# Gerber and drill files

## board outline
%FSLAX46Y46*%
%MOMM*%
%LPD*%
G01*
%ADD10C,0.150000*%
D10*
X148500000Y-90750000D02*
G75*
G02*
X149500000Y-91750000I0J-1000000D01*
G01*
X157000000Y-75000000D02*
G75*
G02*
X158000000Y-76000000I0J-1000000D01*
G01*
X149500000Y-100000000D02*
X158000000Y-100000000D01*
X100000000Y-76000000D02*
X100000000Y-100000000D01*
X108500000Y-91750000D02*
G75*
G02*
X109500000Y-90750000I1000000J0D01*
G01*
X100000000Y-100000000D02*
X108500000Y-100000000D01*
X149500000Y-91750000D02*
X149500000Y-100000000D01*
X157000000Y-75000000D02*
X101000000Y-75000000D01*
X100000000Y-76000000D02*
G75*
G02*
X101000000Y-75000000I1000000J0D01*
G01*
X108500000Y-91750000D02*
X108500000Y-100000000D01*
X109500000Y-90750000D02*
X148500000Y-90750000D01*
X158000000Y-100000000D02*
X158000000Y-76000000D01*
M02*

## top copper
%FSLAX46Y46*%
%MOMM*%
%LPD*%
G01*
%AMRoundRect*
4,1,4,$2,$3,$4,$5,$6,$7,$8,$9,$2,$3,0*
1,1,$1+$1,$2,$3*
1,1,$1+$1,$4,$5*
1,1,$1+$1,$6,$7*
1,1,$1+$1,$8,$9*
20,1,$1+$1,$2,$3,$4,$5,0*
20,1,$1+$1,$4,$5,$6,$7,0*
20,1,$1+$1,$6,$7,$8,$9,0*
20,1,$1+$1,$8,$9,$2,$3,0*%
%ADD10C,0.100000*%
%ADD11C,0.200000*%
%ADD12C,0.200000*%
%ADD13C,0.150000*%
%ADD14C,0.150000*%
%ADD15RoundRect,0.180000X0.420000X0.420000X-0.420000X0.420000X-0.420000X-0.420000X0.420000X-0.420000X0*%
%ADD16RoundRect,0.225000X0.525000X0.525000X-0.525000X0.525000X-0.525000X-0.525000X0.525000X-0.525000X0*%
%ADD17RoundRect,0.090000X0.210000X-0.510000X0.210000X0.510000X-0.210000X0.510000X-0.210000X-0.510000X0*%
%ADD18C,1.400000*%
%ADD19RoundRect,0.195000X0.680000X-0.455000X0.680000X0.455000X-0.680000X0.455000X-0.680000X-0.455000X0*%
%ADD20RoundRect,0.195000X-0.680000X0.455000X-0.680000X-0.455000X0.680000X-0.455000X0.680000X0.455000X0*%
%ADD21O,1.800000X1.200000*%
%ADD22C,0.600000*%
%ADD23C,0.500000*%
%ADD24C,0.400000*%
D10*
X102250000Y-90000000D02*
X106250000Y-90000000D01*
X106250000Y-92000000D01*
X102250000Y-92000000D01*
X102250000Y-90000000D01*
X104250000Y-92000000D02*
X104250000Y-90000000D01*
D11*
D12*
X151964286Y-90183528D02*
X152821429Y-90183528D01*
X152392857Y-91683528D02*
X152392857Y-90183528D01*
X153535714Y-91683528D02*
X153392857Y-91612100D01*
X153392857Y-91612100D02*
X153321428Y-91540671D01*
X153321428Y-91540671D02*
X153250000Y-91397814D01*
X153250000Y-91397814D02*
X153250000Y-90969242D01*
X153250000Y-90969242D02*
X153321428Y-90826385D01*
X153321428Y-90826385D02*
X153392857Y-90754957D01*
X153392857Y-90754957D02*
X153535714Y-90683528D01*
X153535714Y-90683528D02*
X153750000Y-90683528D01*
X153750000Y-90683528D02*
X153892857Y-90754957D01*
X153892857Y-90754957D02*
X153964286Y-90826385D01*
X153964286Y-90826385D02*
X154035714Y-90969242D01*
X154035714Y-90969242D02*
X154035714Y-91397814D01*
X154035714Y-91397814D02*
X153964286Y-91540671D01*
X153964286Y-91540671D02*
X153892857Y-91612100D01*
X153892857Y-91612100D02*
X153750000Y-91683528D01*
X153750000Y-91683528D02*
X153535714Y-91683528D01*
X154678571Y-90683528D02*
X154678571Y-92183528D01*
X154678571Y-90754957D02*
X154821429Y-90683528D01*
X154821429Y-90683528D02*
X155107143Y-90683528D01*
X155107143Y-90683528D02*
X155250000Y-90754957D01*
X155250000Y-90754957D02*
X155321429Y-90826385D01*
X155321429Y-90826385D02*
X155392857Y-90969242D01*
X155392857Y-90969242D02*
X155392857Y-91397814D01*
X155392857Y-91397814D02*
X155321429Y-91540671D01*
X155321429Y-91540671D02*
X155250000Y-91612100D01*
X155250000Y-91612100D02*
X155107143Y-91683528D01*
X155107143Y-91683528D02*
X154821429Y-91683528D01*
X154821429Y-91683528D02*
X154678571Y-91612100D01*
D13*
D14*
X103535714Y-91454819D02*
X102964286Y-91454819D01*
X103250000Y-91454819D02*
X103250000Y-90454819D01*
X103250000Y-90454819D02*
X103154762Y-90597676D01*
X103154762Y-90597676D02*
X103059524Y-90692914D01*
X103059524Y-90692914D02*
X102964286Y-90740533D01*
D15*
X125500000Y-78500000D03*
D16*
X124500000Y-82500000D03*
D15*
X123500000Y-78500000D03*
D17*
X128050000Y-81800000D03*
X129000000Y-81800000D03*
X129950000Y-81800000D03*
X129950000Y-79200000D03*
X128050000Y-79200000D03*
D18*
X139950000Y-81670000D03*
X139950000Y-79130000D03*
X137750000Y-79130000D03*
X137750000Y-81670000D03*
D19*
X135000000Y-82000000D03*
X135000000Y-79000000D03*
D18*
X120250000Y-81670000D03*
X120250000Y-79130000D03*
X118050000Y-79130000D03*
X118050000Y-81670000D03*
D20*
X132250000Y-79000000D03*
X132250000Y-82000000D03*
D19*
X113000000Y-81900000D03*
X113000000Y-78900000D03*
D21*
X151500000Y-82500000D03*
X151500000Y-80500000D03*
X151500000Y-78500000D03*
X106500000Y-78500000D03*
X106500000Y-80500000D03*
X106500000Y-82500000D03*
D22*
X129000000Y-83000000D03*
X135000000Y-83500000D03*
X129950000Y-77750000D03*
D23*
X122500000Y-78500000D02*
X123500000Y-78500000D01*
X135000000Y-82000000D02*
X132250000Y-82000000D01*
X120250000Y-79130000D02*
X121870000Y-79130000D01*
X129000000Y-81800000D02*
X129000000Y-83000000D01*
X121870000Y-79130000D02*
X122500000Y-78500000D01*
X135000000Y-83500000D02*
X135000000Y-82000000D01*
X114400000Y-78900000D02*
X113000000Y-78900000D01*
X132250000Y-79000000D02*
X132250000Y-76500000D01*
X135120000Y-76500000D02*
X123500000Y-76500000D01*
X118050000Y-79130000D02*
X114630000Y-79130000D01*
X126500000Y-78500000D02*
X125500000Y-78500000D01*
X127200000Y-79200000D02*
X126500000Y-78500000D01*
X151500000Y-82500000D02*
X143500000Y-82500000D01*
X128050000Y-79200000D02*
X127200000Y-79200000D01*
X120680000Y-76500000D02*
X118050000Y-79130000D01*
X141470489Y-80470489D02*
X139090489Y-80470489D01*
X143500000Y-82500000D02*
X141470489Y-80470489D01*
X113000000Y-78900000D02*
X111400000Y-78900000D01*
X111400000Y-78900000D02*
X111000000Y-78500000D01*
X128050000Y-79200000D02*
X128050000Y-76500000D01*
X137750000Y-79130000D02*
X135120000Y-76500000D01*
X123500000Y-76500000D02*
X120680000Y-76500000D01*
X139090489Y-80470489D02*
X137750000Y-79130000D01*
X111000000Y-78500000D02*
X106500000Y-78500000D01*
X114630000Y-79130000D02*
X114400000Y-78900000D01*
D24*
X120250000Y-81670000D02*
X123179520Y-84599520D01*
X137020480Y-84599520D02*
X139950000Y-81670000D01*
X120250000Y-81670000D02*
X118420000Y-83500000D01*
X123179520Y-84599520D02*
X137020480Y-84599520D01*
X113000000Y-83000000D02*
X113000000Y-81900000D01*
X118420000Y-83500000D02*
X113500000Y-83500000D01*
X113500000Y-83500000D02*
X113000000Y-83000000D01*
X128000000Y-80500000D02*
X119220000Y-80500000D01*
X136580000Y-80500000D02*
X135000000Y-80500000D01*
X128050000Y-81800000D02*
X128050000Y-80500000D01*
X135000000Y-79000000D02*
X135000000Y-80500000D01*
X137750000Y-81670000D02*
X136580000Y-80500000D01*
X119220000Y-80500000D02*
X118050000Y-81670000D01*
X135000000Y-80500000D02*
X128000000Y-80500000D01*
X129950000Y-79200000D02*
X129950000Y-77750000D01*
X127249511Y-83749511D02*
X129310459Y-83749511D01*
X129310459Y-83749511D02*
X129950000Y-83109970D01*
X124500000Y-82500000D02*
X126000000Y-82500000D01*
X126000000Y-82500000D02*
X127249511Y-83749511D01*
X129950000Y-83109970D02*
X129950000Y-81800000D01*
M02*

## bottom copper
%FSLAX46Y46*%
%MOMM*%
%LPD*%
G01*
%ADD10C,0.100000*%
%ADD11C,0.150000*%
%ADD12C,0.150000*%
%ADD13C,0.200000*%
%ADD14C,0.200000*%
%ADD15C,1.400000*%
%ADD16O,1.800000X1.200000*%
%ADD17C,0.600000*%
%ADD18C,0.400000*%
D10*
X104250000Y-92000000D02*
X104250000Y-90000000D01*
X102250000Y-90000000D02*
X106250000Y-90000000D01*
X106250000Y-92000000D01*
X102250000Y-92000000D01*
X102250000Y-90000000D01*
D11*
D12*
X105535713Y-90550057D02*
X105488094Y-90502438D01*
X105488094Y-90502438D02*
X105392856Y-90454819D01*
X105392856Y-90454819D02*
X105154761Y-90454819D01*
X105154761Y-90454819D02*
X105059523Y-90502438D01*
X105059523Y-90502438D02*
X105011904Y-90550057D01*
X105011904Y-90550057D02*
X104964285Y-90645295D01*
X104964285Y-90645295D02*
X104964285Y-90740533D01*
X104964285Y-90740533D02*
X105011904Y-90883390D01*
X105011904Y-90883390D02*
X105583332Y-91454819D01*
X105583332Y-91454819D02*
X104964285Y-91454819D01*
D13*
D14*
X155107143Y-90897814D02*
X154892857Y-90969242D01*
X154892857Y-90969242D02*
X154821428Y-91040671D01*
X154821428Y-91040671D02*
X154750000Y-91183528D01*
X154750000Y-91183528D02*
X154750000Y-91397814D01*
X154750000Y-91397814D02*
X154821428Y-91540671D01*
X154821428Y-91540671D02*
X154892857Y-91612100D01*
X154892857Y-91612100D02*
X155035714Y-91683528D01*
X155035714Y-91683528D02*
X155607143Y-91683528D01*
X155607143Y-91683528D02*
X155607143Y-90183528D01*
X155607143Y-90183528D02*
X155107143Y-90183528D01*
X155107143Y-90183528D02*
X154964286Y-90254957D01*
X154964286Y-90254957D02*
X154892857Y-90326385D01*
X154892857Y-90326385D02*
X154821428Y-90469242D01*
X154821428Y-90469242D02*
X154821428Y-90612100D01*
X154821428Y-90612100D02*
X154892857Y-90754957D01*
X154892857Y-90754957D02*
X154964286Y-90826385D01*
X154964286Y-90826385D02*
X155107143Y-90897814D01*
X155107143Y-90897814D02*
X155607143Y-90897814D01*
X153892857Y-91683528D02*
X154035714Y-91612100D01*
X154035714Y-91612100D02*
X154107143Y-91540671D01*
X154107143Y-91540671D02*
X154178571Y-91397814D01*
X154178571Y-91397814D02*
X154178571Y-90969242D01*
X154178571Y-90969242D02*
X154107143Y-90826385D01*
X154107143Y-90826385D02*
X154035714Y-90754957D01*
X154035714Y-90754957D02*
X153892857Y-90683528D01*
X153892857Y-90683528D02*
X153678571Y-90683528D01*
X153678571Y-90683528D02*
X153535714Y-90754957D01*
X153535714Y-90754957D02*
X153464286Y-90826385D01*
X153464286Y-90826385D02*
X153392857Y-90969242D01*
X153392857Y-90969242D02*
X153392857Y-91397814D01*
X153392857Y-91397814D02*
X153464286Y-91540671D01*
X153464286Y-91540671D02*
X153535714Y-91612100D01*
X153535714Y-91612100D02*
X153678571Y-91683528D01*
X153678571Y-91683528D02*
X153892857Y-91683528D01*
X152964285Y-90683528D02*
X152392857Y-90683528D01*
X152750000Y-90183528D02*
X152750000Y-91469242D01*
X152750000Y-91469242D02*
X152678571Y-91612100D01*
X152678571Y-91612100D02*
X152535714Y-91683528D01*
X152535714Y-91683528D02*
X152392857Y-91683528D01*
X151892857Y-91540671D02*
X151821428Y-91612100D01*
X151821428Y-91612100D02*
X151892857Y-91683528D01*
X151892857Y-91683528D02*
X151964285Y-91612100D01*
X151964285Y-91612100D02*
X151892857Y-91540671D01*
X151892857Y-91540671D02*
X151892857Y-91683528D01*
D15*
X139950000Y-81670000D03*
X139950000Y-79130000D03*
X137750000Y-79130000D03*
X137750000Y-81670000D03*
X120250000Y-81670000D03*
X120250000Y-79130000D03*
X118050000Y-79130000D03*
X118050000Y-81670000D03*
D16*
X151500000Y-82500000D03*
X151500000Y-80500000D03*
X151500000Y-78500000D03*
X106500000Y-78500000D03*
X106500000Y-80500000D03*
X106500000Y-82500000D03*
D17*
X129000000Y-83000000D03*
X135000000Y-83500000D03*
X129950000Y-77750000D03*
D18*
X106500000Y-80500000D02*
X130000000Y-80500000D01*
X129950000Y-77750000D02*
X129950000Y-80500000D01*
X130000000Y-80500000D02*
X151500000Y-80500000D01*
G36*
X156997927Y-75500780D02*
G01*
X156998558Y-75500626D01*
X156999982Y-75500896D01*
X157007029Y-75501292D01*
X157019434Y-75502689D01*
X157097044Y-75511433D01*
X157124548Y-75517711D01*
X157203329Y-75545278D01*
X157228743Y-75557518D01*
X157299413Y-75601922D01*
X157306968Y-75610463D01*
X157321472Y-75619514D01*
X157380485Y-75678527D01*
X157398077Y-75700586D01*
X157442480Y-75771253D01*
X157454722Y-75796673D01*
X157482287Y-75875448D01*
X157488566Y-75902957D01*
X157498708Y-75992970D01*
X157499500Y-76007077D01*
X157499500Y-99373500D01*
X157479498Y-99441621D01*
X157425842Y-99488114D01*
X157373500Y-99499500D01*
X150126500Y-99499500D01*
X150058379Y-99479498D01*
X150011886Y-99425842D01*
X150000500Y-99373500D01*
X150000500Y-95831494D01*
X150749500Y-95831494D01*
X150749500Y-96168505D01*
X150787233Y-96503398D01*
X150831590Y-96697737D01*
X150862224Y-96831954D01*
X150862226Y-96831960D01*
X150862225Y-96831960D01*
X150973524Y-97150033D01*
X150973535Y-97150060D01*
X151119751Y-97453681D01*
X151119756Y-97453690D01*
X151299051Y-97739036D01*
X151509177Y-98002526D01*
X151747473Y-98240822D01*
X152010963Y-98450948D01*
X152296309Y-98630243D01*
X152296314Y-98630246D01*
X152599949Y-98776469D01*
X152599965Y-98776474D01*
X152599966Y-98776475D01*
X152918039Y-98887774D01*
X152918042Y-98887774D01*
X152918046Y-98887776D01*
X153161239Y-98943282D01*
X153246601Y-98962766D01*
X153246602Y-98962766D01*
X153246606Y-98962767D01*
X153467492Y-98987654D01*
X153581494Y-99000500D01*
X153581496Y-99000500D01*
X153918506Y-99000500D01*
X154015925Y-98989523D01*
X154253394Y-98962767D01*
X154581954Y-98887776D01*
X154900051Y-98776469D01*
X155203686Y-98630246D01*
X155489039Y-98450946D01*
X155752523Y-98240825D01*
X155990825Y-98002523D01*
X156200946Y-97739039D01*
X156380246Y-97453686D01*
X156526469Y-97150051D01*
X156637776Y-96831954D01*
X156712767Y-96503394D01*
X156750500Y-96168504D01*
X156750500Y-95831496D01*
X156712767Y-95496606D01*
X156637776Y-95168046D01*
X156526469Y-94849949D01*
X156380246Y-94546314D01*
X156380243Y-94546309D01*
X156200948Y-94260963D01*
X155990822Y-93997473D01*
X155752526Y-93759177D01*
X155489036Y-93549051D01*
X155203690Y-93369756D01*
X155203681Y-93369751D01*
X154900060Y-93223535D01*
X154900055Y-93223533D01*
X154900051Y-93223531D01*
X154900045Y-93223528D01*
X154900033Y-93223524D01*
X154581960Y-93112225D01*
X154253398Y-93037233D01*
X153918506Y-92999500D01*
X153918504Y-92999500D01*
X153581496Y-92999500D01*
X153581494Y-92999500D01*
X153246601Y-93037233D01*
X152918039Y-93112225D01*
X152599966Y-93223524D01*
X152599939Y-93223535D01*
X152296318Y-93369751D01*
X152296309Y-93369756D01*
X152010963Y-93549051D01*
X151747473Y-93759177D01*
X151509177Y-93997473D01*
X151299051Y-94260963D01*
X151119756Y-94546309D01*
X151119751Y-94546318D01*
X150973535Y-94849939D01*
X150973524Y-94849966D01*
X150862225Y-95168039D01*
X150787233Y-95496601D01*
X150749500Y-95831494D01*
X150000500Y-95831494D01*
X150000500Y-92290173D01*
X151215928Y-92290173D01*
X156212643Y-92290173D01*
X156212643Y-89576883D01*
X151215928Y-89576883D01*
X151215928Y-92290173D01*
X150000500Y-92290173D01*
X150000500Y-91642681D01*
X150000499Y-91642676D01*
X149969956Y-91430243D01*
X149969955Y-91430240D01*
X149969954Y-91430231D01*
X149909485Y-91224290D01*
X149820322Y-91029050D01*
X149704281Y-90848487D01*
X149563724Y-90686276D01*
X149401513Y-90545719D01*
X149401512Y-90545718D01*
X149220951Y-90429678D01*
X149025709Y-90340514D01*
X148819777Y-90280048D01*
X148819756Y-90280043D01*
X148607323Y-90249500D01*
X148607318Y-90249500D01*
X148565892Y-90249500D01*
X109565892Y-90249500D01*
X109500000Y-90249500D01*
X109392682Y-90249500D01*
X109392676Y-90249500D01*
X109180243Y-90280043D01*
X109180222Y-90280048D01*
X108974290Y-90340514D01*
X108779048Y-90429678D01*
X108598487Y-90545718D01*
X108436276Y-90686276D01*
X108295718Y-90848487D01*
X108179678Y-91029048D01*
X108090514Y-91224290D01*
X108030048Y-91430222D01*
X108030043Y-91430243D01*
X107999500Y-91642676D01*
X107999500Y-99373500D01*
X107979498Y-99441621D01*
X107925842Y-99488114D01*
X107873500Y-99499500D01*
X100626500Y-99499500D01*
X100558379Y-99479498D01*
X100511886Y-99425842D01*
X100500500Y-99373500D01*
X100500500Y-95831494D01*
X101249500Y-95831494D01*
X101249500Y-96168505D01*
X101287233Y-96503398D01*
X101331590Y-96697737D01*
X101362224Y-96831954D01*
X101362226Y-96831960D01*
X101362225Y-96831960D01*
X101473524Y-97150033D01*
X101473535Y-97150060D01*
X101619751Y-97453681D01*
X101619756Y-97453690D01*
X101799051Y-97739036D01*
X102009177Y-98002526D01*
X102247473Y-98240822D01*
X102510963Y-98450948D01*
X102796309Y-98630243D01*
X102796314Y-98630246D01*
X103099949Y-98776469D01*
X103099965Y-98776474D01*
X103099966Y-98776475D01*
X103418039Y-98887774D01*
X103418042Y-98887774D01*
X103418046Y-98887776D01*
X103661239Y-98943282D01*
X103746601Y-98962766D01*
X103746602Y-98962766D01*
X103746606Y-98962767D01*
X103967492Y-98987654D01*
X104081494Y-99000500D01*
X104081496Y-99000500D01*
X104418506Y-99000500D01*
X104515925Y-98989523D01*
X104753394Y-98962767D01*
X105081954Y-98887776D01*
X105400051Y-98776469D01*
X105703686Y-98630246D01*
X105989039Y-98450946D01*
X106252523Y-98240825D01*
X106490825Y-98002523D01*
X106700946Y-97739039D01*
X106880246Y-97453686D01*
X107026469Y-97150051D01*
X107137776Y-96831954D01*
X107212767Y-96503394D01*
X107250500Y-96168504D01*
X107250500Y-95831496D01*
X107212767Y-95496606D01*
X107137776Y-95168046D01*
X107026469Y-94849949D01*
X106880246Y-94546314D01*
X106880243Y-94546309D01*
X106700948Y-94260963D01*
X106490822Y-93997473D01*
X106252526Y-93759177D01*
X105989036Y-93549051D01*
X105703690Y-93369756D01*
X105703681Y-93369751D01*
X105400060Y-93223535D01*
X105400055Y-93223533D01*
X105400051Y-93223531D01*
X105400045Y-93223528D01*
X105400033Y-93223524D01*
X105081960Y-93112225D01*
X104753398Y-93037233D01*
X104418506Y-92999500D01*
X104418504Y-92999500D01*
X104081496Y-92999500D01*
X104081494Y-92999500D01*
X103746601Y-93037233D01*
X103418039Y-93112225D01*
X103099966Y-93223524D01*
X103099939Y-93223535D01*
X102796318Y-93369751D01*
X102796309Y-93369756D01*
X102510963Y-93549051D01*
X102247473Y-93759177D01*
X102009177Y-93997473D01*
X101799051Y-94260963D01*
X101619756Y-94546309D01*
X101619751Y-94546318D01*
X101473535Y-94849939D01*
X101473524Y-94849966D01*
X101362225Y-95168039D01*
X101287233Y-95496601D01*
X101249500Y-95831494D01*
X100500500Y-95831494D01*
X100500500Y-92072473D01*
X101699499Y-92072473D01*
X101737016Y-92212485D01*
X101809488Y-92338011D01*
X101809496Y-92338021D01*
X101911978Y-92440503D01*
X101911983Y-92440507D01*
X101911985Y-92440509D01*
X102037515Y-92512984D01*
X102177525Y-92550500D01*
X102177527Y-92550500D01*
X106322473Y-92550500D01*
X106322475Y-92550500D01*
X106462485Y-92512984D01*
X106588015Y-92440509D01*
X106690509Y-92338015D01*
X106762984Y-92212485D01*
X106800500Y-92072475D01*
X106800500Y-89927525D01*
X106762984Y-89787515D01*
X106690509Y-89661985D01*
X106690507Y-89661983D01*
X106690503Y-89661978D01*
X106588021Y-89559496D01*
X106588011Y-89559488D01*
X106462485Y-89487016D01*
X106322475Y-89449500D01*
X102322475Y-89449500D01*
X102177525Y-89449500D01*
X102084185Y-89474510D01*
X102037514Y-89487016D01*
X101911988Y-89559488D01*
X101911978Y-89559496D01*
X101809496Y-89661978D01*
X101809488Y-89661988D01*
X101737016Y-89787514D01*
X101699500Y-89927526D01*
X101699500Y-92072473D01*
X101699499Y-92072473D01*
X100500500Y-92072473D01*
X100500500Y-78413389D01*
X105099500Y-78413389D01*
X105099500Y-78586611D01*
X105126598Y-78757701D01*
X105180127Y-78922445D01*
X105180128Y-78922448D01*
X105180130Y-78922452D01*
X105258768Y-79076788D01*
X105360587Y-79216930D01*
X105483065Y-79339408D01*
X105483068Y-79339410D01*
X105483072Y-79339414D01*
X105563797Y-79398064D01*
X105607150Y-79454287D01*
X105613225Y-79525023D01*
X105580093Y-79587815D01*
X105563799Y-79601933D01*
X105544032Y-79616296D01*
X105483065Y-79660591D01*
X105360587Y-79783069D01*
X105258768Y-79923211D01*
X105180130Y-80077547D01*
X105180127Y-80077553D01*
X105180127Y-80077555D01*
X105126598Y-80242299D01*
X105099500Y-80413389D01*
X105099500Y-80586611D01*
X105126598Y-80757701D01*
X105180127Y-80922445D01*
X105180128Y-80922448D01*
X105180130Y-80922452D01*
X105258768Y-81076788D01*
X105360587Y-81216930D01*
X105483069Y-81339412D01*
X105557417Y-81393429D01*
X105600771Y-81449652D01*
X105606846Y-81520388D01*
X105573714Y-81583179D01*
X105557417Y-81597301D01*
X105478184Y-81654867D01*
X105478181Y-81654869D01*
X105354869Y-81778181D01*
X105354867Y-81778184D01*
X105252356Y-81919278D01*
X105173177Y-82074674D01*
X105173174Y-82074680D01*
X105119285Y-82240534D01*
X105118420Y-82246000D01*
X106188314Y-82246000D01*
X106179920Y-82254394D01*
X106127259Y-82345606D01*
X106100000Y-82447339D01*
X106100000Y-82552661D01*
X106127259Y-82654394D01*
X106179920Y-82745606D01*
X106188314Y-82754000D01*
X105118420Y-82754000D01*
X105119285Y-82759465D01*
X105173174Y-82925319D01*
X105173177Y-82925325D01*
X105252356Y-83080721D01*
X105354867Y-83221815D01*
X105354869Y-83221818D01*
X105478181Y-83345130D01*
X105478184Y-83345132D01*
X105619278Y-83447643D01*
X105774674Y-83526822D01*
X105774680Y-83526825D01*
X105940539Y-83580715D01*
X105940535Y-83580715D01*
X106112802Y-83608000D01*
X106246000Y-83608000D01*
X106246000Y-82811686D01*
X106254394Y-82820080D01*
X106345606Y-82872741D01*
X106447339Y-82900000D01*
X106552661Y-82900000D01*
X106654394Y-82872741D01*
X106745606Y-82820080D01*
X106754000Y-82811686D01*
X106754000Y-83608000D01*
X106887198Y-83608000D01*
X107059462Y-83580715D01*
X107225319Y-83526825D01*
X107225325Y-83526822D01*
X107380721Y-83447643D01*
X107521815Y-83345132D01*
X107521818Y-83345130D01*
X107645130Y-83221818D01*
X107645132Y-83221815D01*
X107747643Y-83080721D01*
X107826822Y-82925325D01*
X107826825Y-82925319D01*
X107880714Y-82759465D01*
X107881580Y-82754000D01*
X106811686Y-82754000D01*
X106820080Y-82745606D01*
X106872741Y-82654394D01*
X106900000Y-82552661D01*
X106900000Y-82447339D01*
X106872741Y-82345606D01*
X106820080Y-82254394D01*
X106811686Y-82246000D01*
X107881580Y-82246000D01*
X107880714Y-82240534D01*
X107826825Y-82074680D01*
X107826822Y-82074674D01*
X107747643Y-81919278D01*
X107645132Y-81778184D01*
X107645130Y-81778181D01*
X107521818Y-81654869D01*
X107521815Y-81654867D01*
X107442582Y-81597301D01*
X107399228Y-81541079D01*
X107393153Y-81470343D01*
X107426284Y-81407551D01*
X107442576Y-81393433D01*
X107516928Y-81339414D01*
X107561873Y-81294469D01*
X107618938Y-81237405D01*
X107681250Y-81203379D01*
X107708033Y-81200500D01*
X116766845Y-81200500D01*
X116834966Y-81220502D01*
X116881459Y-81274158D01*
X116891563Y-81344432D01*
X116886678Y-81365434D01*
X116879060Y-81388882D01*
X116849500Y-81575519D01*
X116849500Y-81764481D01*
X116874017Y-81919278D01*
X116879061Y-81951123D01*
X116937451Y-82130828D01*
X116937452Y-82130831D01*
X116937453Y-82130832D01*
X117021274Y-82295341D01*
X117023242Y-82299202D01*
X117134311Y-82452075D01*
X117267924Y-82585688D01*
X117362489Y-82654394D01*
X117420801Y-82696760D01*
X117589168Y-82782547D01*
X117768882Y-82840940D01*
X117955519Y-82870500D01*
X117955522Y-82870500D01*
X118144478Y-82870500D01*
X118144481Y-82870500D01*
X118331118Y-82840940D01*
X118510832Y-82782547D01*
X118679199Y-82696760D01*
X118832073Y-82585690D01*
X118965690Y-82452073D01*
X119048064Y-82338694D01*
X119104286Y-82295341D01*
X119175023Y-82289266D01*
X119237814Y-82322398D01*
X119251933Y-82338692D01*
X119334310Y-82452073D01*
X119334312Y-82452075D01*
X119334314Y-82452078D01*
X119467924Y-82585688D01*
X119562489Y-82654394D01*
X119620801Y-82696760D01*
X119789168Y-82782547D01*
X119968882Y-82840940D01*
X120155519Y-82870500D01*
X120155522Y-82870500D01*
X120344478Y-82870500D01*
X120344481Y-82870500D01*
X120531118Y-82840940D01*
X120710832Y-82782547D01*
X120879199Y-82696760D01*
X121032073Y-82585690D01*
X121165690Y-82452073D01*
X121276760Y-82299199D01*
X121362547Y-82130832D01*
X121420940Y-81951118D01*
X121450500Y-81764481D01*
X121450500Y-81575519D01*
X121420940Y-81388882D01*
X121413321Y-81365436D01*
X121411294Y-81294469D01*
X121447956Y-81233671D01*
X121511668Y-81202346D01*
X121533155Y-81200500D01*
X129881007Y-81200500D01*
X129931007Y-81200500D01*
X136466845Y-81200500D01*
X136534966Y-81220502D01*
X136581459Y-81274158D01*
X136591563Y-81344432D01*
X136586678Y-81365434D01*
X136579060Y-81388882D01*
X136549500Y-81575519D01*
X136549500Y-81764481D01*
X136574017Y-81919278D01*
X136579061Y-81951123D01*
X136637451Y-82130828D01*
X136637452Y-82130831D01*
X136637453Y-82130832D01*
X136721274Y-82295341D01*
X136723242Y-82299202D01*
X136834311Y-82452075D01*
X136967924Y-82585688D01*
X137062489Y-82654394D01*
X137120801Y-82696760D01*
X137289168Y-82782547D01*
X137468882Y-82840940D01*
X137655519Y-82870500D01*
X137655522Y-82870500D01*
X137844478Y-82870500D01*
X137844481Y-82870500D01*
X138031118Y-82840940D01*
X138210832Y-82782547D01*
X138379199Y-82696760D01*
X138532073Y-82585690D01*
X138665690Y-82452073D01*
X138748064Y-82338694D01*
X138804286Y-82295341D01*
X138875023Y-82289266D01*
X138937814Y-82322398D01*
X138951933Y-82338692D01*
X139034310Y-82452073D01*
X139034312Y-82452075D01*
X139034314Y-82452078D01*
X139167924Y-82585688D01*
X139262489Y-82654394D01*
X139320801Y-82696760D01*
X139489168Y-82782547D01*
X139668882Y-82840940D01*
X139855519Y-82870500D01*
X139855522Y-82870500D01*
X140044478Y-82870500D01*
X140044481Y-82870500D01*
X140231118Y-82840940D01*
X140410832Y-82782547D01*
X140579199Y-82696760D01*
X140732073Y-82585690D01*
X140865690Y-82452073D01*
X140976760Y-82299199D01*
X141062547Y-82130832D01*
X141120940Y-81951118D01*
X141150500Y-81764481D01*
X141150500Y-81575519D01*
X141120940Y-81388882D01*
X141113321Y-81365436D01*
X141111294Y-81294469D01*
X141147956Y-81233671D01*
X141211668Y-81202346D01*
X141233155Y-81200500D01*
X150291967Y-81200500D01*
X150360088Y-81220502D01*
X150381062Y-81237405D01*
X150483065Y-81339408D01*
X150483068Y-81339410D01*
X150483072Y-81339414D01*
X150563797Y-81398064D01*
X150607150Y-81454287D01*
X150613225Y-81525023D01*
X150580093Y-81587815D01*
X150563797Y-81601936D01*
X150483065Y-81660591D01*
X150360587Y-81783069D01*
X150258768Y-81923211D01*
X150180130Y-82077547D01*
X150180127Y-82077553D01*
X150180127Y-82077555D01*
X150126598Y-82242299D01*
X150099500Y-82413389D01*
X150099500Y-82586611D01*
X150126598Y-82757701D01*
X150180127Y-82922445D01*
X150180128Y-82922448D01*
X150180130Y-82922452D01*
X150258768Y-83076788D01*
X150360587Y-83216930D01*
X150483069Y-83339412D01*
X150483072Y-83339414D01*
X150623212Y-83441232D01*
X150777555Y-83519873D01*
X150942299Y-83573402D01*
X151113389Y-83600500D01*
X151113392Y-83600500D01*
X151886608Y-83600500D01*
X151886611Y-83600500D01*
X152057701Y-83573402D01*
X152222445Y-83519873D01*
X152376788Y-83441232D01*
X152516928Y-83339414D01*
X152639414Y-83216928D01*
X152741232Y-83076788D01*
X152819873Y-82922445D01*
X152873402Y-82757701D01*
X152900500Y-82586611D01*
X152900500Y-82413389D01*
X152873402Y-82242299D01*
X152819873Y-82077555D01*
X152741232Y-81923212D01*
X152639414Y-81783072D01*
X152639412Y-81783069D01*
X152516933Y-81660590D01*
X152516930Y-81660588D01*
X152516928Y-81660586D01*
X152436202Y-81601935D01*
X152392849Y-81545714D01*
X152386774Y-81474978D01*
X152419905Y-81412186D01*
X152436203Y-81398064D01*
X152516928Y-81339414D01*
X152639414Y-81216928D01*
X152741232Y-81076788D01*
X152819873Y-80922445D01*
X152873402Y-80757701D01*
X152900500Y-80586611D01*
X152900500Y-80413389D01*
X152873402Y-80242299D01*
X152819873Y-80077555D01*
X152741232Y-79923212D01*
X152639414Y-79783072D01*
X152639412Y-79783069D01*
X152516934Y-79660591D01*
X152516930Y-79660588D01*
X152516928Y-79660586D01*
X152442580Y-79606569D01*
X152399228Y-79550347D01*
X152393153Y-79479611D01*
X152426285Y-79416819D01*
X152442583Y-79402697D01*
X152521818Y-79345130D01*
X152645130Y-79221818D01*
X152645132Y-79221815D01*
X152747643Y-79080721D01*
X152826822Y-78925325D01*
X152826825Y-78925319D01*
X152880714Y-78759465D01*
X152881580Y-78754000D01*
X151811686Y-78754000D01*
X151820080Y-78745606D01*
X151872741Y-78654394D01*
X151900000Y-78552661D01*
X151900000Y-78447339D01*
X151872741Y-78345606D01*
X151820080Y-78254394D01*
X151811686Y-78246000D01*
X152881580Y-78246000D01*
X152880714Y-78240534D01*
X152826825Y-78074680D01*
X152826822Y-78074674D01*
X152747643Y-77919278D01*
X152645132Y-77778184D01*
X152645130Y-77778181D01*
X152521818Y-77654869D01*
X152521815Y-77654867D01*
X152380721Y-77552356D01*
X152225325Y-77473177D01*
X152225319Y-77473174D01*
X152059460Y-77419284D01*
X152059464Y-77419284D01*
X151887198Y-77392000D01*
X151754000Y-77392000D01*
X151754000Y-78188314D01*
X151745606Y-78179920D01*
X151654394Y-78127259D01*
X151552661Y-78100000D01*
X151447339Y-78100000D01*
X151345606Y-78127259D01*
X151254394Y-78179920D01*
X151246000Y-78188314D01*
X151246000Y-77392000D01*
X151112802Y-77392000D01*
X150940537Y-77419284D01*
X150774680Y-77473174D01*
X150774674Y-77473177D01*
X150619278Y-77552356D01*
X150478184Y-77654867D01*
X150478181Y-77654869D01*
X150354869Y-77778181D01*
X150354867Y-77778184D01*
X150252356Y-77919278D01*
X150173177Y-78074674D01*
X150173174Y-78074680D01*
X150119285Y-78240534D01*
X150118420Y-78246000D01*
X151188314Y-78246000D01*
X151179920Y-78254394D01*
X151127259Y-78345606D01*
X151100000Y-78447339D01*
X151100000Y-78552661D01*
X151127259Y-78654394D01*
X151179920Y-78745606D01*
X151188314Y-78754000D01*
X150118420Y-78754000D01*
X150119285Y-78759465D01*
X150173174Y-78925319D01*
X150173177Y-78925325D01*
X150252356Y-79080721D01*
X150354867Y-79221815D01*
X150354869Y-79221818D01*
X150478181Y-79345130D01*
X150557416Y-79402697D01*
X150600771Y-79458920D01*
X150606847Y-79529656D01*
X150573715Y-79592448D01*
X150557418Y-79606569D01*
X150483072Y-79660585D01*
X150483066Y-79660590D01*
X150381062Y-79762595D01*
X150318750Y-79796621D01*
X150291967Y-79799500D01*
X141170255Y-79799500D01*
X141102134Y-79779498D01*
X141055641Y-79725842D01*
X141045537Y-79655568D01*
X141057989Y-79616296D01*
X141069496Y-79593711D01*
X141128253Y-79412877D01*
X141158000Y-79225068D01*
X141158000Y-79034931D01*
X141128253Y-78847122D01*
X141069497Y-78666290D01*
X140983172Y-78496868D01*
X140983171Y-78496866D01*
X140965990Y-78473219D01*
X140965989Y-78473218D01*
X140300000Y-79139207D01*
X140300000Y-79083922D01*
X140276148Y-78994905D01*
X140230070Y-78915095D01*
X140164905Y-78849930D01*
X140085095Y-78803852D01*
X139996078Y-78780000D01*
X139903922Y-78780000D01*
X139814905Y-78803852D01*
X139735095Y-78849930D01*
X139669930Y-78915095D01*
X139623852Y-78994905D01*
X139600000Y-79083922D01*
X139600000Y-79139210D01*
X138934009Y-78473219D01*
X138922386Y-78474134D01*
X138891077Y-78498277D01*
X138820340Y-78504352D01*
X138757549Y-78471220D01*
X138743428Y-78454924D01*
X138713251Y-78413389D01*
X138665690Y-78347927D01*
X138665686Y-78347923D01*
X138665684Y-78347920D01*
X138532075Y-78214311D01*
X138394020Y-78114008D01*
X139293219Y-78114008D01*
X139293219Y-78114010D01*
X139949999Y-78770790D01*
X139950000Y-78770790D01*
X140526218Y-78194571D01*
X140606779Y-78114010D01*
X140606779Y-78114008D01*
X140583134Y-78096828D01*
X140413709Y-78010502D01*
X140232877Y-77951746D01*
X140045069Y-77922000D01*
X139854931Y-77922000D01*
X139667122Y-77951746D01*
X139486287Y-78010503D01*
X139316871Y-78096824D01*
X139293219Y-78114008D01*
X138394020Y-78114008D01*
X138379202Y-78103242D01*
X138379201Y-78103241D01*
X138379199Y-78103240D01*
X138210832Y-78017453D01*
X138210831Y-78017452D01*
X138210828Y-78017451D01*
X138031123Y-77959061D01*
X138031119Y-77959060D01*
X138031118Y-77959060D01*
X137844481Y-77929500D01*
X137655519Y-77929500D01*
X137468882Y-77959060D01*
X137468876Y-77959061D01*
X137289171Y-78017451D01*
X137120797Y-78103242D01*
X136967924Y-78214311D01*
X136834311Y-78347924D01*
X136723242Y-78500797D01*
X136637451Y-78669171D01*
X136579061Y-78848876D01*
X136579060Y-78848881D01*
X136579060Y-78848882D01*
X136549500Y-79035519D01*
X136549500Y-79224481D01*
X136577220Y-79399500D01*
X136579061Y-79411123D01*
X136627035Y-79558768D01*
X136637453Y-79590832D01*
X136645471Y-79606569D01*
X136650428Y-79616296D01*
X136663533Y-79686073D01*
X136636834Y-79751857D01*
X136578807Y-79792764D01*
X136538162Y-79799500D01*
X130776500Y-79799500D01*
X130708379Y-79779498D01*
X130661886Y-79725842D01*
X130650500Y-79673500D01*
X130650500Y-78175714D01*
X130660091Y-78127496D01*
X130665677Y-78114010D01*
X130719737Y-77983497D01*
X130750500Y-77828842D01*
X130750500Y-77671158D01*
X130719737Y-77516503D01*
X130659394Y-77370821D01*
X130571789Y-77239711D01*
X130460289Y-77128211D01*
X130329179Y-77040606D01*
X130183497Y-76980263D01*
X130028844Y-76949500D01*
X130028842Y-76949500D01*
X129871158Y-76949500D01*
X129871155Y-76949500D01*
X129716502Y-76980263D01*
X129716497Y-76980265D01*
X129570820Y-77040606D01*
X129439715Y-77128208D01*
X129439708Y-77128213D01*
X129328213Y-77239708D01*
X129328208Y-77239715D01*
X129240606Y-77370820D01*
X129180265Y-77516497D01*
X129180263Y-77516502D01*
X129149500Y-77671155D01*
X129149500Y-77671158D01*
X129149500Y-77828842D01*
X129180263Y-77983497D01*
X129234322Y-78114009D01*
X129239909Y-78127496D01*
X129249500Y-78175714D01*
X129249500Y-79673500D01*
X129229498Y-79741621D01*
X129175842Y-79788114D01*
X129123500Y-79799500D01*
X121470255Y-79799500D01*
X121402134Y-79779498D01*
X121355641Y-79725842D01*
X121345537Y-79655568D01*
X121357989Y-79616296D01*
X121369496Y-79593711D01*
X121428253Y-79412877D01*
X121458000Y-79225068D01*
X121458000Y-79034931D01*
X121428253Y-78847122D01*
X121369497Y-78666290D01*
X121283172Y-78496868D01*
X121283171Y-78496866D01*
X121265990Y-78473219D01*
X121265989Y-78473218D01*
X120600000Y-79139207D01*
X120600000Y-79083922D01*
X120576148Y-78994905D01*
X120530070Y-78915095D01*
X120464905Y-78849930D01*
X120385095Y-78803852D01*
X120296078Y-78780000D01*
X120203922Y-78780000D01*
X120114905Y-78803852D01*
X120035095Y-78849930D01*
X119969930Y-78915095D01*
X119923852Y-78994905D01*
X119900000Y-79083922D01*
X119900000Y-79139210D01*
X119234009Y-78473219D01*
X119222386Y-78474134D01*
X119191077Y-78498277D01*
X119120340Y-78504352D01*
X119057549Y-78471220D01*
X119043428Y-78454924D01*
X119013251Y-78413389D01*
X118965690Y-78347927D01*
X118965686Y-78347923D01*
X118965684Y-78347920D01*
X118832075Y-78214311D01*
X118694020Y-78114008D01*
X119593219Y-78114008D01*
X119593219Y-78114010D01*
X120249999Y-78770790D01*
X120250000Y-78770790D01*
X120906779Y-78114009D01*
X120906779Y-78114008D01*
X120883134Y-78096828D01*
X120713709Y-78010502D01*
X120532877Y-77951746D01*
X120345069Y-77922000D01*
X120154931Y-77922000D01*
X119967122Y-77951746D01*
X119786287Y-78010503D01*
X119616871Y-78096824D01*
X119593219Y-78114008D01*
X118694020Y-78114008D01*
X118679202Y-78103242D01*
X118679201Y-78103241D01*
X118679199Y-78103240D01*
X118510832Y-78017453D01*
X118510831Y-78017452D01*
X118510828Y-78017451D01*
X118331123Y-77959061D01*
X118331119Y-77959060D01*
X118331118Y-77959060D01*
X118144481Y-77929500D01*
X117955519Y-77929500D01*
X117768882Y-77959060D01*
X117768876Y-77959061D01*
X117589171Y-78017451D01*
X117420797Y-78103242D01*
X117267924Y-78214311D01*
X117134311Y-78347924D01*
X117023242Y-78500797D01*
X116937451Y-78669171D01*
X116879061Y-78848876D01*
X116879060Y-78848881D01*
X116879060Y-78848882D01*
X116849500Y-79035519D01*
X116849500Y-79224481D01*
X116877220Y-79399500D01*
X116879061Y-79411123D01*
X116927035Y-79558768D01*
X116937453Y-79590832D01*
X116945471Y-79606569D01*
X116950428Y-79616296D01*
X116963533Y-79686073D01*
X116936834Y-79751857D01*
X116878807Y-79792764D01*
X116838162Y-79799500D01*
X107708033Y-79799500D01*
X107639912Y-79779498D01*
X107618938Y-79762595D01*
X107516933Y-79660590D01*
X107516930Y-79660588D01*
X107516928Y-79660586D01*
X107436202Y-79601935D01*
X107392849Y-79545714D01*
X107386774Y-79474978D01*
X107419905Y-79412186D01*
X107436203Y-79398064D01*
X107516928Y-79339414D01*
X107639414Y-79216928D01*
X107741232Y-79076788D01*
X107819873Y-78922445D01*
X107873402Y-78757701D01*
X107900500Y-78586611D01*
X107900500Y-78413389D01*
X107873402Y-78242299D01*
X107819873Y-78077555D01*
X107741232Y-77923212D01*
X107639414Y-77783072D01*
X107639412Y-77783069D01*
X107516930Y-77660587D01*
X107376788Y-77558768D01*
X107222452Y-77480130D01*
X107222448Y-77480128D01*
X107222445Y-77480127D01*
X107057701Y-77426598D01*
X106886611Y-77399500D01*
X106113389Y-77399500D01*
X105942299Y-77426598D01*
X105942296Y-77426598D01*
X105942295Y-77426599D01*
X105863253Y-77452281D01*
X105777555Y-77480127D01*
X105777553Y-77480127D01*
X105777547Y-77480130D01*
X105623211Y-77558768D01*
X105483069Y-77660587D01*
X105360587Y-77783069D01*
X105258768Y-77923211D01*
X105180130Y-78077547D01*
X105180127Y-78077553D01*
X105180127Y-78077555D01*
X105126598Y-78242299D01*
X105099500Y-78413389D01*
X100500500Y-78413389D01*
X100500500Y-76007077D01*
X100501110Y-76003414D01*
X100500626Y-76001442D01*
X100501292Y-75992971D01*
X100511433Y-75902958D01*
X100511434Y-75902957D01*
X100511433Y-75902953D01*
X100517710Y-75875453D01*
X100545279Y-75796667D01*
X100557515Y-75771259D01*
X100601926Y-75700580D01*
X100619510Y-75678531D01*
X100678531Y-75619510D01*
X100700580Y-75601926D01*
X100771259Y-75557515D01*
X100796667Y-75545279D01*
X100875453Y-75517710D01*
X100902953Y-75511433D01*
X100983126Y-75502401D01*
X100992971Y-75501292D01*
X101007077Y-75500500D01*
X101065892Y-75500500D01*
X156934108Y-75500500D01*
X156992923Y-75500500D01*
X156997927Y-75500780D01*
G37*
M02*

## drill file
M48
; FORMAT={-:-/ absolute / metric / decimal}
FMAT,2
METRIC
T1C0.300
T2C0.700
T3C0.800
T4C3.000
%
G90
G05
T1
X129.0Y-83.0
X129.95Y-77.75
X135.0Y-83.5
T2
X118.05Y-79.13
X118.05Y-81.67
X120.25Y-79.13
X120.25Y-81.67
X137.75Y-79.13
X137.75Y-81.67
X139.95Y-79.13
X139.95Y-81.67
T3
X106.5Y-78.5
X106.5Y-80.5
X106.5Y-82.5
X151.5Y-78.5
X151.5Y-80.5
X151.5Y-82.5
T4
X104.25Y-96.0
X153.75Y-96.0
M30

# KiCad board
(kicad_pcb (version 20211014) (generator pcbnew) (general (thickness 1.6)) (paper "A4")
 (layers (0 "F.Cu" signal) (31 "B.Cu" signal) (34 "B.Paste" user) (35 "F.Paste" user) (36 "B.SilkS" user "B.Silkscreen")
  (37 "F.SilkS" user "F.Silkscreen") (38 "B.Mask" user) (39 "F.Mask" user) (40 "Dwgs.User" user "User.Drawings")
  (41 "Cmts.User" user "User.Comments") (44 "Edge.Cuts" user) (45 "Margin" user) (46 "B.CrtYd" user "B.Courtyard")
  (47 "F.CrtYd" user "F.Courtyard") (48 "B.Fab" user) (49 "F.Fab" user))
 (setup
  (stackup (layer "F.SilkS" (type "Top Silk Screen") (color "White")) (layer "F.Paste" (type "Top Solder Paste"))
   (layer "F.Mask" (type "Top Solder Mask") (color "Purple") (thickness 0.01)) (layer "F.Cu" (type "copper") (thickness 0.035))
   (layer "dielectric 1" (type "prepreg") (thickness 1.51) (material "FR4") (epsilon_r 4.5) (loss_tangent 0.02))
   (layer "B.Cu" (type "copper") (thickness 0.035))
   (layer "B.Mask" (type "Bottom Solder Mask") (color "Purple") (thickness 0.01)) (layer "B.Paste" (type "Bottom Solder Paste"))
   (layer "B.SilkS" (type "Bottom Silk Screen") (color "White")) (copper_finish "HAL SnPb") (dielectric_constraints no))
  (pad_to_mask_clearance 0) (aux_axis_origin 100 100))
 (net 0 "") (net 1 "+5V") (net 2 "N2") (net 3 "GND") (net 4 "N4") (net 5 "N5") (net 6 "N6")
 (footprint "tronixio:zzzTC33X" (layer "F.Cu") (at 124.5 80.5 180) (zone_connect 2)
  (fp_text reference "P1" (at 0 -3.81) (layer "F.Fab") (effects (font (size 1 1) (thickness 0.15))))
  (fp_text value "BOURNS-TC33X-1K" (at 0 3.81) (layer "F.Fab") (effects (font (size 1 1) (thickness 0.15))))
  (pad "1" smd roundrect (at -1 2 180) (size 1.2 1.2) (layers "F.Cu" "F.Paste" "F.Mask") (roundrect_rratio 0.15) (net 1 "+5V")
   (zone_connect 2))
  (pad "2" smd roundrect (at 0 -2 180) (size 1.5 1.5) (layers "F.Cu" "F.Paste" "F.Mask") (roundrect_rratio 0.15) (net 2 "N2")
   (zone_connect 2))
  (pad "3" smd roundrect (at 1 2 180) (size 1.2 1.2) (layers "F.Cu" "F.Paste" "F.Mask") (roundrect_rratio 0.15) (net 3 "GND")
   (zone_connect 2)))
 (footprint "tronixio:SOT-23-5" (layer "F.Cu") (at 129 80.5 90)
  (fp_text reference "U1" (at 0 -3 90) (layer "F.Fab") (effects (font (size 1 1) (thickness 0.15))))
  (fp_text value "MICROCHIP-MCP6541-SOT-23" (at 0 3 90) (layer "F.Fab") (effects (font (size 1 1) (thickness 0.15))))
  (pad "1" smd roundrect (at -1.3 -0.95 90) (size 1.2 0.6) (layers "F.Cu" "F.Paste" "F.Mask") (roundrect_rratio 0.15) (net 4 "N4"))
  (pad "2" smd roundrect (at -1.3 0 90) (size 1.2 0.6) (layers "F.Cu" "F.Paste" "F.Mask") (roundrect_rratio 0.15) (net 3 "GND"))
  (pad "3" smd roundrect (at -1.3 0.95 90) (size 1.2 0.6) (layers "F.Cu" "F.Paste" "F.Mask") (roundrect_rratio 0.15) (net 2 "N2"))
  (pad "4" smd roundrect (at 1.3 0.95 90) (size 1.2 0.6) (layers "F.Cu" "F.Paste" "F.Mask") (roundrect_rratio 0.15) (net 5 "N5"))
  (pad "5" smd roundrect (at 1.3 -0.95 90) (size 1.2 0.6) (layers "F.Cu" "F.Paste" "F.Mask") (roundrect_rratio 0.15) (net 1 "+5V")))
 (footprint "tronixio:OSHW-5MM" (layer "F.Cu") (at 129 87.5)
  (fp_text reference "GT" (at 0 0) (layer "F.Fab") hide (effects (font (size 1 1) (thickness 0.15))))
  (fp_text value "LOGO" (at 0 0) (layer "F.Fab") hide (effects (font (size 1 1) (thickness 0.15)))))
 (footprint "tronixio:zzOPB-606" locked (layer "F.Cu") (at 138.85 80.4)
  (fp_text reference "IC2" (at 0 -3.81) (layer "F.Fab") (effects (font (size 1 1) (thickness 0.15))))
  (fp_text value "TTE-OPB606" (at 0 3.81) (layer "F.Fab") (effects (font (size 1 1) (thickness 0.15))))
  (pad "1" thru_hole circle locked (at 1.1 1.27) (size 1.4 1.4) (drill 0.7) (layers *.Cu *.Mask) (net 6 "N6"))
  (pad "2" thru_hole circle locked (at 1.1 -1.27) (size 1.4 1.4) (drill 0.7) (layers *.Cu *.Mask) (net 3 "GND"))
  (pad "3" thru_hole circle locked (at -1.1 -1.27) (size 1.4 1.4) (drill 0.7) (layers *.Cu *.Mask) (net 1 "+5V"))
  (pad "4" thru_hole circle locked (at -1.1 1.27) (size 1.4 1.4) (drill 0.7) (layers *.Cu *.Mask) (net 4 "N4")))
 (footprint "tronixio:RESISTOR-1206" (layer "F.Cu") (at 135 80.5 90) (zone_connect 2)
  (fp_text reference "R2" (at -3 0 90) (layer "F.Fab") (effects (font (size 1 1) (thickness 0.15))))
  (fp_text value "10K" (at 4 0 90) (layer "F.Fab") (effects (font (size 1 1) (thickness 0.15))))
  (pad "1" smd roundrect (at -1.5 0 90) (size 1.3 1.75) (layers "F.Cu" "F.Paste" "F.Mask") (roundrect_rratio 0.15) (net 3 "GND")
   (zone_connect 1))
  (pad "2" smd roundrect (at 1.5 0 90) (size 1.3 1.75) (layers "F.Cu" "F.Paste" "F.Mask") (roundrect_rratio 0.15) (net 4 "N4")
   (zone_connect 2)))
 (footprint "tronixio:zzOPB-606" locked (layer "F.Cu") (at 119.15 80.4)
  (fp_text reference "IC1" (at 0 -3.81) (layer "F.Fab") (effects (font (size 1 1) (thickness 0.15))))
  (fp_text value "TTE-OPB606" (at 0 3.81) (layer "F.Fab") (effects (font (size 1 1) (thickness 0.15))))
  (pad "1" thru_hole circle locked (at 1.1 1.27) (size 1.4 1.4) (drill 0.7) (layers *.Cu *.Mask) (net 6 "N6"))
  (pad "2" thru_hole circle locked (at 1.1 -1.27) (size 1.4 1.4) (drill 0.7) (layers *.Cu *.Mask) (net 3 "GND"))
  (pad "3" thru_hole circle locked (at -1.1 -1.27) (size 1.4 1.4) (drill 0.7) (layers *.Cu *.Mask) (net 1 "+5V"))
  (pad "4" thru_hole circle locked (at -1.1 1.27) (size 1.4 1.4) (drill 0.7) (layers *.Cu *.Mask) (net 4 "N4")))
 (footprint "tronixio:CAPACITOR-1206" (layer "F.Cu") (at 132.25 80.5 -90) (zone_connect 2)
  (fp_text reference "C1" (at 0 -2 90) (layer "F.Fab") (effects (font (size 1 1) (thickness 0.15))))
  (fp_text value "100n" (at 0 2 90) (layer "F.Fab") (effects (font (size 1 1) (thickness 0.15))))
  (pad "1" smd roundrect (at -1.5 0 270) (size 1.3 1.75) (layers "F.Cu" "F.Paste" "F.Mask") (roundrect_rratio 0.15) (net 1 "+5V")
   (zone_connect 2))
  (pad "2" smd roundrect (at 1.5 0 270) (size 1.3 1.75) (layers "F.Cu" "F.Paste" "F.Mask") (roundrect_rratio 0.15) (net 3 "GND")
   (zone_connect 1)))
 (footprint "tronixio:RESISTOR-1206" (layer "F.Cu") (at 113 80.4 90) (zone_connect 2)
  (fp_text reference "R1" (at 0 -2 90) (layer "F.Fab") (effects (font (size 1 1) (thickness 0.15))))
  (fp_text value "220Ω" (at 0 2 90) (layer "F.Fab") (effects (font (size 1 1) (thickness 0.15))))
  (pad "1" smd roundrect (at -1.5 0 90) (size 1.3 1.75) (layers "F.Cu" "F.Paste" "F.Mask") (roundrect_rratio 0.15) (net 6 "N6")
   (zone_connect 2))
  (pad "2" smd roundrect (at 1.5 0 90) (size 1.3 1.75) (layers "F.Cu" "F.Paste" "F.Mask") (roundrect_rratio 0.15) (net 1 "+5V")
   (zone_connect 2)))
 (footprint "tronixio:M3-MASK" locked (layer "B.Cu") (at 153.75 96 180)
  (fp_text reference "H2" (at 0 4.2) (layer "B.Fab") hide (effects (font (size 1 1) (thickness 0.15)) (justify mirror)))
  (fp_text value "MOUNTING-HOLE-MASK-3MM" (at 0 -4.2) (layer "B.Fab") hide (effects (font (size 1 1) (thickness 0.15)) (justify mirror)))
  (pad "" np_thru_hole circle locked (at 0 0 180) (size 3 3) (drill 3) (layers F&B.Cu *.Mask) (solder_mask_margin 1.5) (clearance 1.5)))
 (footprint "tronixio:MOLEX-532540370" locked (layer "B.Cu") (at 151.5 82.5 90)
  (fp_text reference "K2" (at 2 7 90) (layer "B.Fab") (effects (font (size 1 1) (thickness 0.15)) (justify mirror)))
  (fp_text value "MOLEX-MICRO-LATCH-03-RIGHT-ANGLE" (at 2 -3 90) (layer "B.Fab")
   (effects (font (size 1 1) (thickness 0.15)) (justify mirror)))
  (pad "1" thru_hole oval locked (at 0 0 90) (size 1.2 1.8) (drill 0.8) (layers *.Cu *.Mask) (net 1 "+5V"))
  (pad "2" thru_hole oval locked (at 2 0 90) (size 1.2 1.8) (drill 0.8) (layers *.Cu *.Mask) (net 5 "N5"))
  (pad "3" thru_hole oval locked (at 4 0 90) (size 1.2 1.8) (drill 0.8) (layers *.Cu *.Mask) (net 3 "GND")))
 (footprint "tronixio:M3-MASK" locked (layer "B.Cu") (at 104.25 96 90)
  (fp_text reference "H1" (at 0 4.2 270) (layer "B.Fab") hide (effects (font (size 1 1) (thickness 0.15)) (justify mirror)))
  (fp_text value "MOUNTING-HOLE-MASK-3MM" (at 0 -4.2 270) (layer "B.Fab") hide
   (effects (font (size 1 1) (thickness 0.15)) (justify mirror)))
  (pad "" np_thru_hole circle locked (at 0 0 90) (size 3 3) (drill 3) (layers F&B.Cu *.Mask) (solder_mask_margin 1.5) (clearance 1.5)))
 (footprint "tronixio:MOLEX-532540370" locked (layer "B.Cu") (at 106.5 78.5 -90)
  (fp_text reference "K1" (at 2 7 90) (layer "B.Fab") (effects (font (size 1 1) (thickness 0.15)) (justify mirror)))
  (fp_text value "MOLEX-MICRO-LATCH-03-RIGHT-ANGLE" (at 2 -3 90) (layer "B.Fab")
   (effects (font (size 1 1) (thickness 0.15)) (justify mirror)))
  (pad "1" thru_hole oval locked (at 0 0 270) (size 1.2 1.8) (drill 0.8) (layers *.Cu *.Mask) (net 1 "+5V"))
  (pad "2" thru_hole oval locked (at 2 0 270) (size 1.2 1.8) (drill 0.8) (layers *.Cu *.Mask) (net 5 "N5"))
  (pad "3" thru_hole oval locked (at 4 0 270) (size 1.2 1.8) (drill 0.8) (layers *.Cu *.Mask) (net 3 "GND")))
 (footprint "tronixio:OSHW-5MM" (layer "B.Cu") (at 129 87.5 180)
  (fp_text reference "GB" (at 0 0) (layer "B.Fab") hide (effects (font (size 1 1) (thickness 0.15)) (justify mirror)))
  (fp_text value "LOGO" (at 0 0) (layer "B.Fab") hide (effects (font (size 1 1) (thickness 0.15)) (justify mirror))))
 (gr_rect (start 102.25 92) (end 106.25 90) (layer "F.Cu") (width 0.1) (fill none))
 (gr_line (start 104.25 92) (end 104.25 90) (layer "F.Cu") (width 0.1))
 (gr_line (start 104.25 92) (end 104.25 90) (layer "B.Cu") (width 0.1))
 (gr_rect (start 102.25 92) (end 106.25 90) (layer "B.Cu") (width 0.1) (fill none))
 (gr_arc (start 148.5 90.75) (mid 149.207107 91.042893) (end 149.5 91.75) (layer "Edge.Cuts") (width 0.15))
 (gr_arc (start 157 75) (mid 157.707107 75.292893) (end 158 76) (layer "Edge.Cuts") (width 0.15))
 (gr_line (start 149.5 100) (end 158 100) (layer "Edge.Cuts") (width 0.15))
 (gr_line (start 100 76) (end 100 100) (layer "Edge.Cuts") (width 0.15))
 (gr_arc (start 108.5 91.75) (mid 108.792893 91.042893) (end 109.5 90.75) (layer "Edge.Cuts") (width 0.15))
 (gr_line (start 100 100) (end 108.5 100) (layer "Edge.Cuts") (width 0.15))
 (gr_line (start 149.5 91.75) (end 149.5 100) (layer "Edge.Cuts") (width 0.15))
 (gr_line (start 157 75) (end 101 75) (layer "Edge.Cuts") (width 0.15))
 (gr_arc (start 100 76) (mid 100.292893 75.292893) (end 101 75) (layer "Edge.Cuts") (width 0.15))
 (gr_line (start 108.5 91.75) (end 108.5 100) (layer "Edge.Cuts") (width 0.15))
 (gr_line (start 109.5 90.75) (end 148.5 90.75) (layer "Edge.Cuts") (width 0.15))
 (gr_line (start 158 100) (end 158 76) (layer "Edge.Cuts") (width 0.15))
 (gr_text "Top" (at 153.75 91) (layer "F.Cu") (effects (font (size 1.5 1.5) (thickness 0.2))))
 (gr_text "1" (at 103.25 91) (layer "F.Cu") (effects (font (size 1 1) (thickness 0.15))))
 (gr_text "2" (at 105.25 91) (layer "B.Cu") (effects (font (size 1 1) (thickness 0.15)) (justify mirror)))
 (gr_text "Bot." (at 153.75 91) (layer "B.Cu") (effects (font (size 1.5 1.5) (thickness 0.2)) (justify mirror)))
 (segment (start 122.5 78.5) (end 123.5 78.5) (width 0.5) (layer "F.Cu") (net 3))
 (segment (start 135 82) (end 132.25 82) (width 0.5) (layer "F.Cu") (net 3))
 (segment (start 120.25 79.13) (end 121.87 79.13) (width 0.5) (layer "F.Cu") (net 3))
 (segment (start 129 81.8) (end 129 83) (width 0.5) (layer "F.Cu") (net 3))
 (segment (start 121.87 79.13) (end 122.5 78.5) (width 0.5) (layer "F.Cu") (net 3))
 (segment (start 135 83.5) (end 135 82) (width 0.5) (layer "F.Cu") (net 3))
 (via (at 129 83) (size 0.6) (drill 0.3) (layers "F.Cu" "B.Cu") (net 3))
 (via (at 135 83.5) (size 0.6) (drill 0.3) (layers "F.Cu" "B.Cu") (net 3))
 (segment (start 114.4 78.9) (end 113 78.9) (width 0.5) (layer "F.Cu") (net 1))
 (segment (start 132.25 79) (end 132.25 76.5) (width 0.5) (layer "F.Cu") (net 1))
 (segment (start 135.12 76.5) (end 123.5 76.5) (width 0.5) (layer "F.Cu") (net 1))
 (segment (start 118.05 79.13) (end 114.63 79.13) (width 0.5) (layer "F.Cu") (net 1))
 (segment (start 126.5 78.5) (end 125.5 78.5) (width 0.5) (layer "F.Cu") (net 1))
 (segment (start 127.2 79.2) (end 126.5 78.5) (width 0.5) (layer "F.Cu") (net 1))
 (segment (start 151.5 82.5) (end 143.5 82.5) (width 0.5) (layer "F.Cu") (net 1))
 (segment (start 128.05 79.2) (end 127.2 79.2) (width 0.5) (layer "F.Cu") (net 1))
 (segment (start 120.68 76.5) (end 118.05 79.13) (width 0.5) (layer "F.Cu") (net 1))
 (segment (start 141.470489 80.470489) (end 139.090489 80.470489) (width 0.5) (layer "F.Cu") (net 1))
 (segment (start 143.5 82.5) (end 141.470489 80.470489) (width 0.5) (layer "F.Cu") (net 1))
 (segment (start 113 78.9) (end 111.4 78.9) (width 0.5) (layer "F.Cu") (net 1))
 (segment (start 111.4 78.9) (end 111 78.5) (width 0.5) (layer "F.Cu") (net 1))
 (segment (start 128.05 79.2) (end 128.05 76.5) (width 0.5) (layer "F.Cu") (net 1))
 (segment (start 137.75 79.13) (end 135.12 76.5) (width 0.5) (layer "F.Cu") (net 1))
 (segment (start 123.5 76.5) (end 120.68 76.5) (width 0.5) (layer "F.Cu") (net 1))
 (segment (start 139.090489 80.470489) (end 137.75 79.13) (width 0.5) (layer "F.Cu") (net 1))
 (segment (start 111 78.5) (end 106.5 78.5) (width 0.5) (layer "F.Cu") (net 1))
 (segment (start 114.63 79.13) (end 114.4 78.9) (width 0.5) (layer "F.Cu") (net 1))
 (segment (start 120.25 81.67) (end 123.17952 84.59952) (width 0.4) (layer "F.Cu") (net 6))
 (segment (start 137.02048 84.59952) (end 139.95 81.67) (width 0.4) (layer "F.Cu") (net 6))
 (segment (start 120.25 81.67) (end 118.42 83.5) (width 0.4) (layer "F.Cu") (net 6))
 (segment (start 123.17952 84.59952) (end 137.02048 84.59952) (width 0.4) (layer "F.Cu") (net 6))
 (segment (start 113 83) (end 113 81.9) (width 0.4) (layer "F.Cu") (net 6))
 (segment (start 118.42 83.5) (end 113.5 83.5) (width 0.4) (layer "F.Cu") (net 6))
 (segment (start 113.5 83.5) (end 113 83) (width 0.4) (layer "F.Cu") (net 6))
 (segment (start 128 80.5) (end 119.22 80.5) (width 0.4) (layer "F.Cu") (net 4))
 (segment (start 136.58 80.5) (end 135 80.5) (width 0.4) (layer "F.Cu") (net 4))
 (segment (start 128.05 81.8) (end 128.05 80.5) (width 0.4) (layer "F.Cu") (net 4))
 (segment (start 135 79) (end 135 80.5) (width 0.4) (layer "F.Cu") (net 4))
 (segment (start 137.75 81.67) (end 136.58 80.5) (width 0.4) (layer "F.Cu") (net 4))
 (segment (start 119.22 80.5) (end 118.05 81.67) (width 0.4) (layer "F.Cu") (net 4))
 (segment (start 135 80.5) (end 128 80.5) (width 0.4) (layer "F.Cu") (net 4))
 (segment (start 129.95 79.2) (end 129.95 77.75) (width 0.4) (layer "F.Cu") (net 5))
 (via (at 129.95 77.75) (size 0.6) (drill 0.3) (layers "F.Cu" "B.Cu") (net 5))
 (segment (start 106.5 80.5) (end 130 80.5) (width 0.4) (layer "B.Cu") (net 5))
 (segment (start 129.95 77.75) (end 129.95 80.5) (width 0.4) (layer "B.Cu") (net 5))
 (segment (start 130 80.5) (end 151.5 80.5) (width 0.4) (layer "B.Cu") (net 5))
 (segment (start 127.249511 83.749511) (end 129.310459 83.749511) (width 0.4) (layer "F.Cu") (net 2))
 (segment (start 129.310459 83.749511) (end 129.95 83.10997) (width 0.4) (layer "F.Cu") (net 2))
 (segment (start 124.5 82.5) (end 126 82.5) (width 0.4) (layer "F.Cu") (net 2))
 (segment (start 126 82.5) (end 127.249511 83.749511) (width 0.4) (layer "F.Cu") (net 2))
 (segment (start 129.95 83.10997) (end 129.95 81.8) (width 0.4) (layer "F.Cu") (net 2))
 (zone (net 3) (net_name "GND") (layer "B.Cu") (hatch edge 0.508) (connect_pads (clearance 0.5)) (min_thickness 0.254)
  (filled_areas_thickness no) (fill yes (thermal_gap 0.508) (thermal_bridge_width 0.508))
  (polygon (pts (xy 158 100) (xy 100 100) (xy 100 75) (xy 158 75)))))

